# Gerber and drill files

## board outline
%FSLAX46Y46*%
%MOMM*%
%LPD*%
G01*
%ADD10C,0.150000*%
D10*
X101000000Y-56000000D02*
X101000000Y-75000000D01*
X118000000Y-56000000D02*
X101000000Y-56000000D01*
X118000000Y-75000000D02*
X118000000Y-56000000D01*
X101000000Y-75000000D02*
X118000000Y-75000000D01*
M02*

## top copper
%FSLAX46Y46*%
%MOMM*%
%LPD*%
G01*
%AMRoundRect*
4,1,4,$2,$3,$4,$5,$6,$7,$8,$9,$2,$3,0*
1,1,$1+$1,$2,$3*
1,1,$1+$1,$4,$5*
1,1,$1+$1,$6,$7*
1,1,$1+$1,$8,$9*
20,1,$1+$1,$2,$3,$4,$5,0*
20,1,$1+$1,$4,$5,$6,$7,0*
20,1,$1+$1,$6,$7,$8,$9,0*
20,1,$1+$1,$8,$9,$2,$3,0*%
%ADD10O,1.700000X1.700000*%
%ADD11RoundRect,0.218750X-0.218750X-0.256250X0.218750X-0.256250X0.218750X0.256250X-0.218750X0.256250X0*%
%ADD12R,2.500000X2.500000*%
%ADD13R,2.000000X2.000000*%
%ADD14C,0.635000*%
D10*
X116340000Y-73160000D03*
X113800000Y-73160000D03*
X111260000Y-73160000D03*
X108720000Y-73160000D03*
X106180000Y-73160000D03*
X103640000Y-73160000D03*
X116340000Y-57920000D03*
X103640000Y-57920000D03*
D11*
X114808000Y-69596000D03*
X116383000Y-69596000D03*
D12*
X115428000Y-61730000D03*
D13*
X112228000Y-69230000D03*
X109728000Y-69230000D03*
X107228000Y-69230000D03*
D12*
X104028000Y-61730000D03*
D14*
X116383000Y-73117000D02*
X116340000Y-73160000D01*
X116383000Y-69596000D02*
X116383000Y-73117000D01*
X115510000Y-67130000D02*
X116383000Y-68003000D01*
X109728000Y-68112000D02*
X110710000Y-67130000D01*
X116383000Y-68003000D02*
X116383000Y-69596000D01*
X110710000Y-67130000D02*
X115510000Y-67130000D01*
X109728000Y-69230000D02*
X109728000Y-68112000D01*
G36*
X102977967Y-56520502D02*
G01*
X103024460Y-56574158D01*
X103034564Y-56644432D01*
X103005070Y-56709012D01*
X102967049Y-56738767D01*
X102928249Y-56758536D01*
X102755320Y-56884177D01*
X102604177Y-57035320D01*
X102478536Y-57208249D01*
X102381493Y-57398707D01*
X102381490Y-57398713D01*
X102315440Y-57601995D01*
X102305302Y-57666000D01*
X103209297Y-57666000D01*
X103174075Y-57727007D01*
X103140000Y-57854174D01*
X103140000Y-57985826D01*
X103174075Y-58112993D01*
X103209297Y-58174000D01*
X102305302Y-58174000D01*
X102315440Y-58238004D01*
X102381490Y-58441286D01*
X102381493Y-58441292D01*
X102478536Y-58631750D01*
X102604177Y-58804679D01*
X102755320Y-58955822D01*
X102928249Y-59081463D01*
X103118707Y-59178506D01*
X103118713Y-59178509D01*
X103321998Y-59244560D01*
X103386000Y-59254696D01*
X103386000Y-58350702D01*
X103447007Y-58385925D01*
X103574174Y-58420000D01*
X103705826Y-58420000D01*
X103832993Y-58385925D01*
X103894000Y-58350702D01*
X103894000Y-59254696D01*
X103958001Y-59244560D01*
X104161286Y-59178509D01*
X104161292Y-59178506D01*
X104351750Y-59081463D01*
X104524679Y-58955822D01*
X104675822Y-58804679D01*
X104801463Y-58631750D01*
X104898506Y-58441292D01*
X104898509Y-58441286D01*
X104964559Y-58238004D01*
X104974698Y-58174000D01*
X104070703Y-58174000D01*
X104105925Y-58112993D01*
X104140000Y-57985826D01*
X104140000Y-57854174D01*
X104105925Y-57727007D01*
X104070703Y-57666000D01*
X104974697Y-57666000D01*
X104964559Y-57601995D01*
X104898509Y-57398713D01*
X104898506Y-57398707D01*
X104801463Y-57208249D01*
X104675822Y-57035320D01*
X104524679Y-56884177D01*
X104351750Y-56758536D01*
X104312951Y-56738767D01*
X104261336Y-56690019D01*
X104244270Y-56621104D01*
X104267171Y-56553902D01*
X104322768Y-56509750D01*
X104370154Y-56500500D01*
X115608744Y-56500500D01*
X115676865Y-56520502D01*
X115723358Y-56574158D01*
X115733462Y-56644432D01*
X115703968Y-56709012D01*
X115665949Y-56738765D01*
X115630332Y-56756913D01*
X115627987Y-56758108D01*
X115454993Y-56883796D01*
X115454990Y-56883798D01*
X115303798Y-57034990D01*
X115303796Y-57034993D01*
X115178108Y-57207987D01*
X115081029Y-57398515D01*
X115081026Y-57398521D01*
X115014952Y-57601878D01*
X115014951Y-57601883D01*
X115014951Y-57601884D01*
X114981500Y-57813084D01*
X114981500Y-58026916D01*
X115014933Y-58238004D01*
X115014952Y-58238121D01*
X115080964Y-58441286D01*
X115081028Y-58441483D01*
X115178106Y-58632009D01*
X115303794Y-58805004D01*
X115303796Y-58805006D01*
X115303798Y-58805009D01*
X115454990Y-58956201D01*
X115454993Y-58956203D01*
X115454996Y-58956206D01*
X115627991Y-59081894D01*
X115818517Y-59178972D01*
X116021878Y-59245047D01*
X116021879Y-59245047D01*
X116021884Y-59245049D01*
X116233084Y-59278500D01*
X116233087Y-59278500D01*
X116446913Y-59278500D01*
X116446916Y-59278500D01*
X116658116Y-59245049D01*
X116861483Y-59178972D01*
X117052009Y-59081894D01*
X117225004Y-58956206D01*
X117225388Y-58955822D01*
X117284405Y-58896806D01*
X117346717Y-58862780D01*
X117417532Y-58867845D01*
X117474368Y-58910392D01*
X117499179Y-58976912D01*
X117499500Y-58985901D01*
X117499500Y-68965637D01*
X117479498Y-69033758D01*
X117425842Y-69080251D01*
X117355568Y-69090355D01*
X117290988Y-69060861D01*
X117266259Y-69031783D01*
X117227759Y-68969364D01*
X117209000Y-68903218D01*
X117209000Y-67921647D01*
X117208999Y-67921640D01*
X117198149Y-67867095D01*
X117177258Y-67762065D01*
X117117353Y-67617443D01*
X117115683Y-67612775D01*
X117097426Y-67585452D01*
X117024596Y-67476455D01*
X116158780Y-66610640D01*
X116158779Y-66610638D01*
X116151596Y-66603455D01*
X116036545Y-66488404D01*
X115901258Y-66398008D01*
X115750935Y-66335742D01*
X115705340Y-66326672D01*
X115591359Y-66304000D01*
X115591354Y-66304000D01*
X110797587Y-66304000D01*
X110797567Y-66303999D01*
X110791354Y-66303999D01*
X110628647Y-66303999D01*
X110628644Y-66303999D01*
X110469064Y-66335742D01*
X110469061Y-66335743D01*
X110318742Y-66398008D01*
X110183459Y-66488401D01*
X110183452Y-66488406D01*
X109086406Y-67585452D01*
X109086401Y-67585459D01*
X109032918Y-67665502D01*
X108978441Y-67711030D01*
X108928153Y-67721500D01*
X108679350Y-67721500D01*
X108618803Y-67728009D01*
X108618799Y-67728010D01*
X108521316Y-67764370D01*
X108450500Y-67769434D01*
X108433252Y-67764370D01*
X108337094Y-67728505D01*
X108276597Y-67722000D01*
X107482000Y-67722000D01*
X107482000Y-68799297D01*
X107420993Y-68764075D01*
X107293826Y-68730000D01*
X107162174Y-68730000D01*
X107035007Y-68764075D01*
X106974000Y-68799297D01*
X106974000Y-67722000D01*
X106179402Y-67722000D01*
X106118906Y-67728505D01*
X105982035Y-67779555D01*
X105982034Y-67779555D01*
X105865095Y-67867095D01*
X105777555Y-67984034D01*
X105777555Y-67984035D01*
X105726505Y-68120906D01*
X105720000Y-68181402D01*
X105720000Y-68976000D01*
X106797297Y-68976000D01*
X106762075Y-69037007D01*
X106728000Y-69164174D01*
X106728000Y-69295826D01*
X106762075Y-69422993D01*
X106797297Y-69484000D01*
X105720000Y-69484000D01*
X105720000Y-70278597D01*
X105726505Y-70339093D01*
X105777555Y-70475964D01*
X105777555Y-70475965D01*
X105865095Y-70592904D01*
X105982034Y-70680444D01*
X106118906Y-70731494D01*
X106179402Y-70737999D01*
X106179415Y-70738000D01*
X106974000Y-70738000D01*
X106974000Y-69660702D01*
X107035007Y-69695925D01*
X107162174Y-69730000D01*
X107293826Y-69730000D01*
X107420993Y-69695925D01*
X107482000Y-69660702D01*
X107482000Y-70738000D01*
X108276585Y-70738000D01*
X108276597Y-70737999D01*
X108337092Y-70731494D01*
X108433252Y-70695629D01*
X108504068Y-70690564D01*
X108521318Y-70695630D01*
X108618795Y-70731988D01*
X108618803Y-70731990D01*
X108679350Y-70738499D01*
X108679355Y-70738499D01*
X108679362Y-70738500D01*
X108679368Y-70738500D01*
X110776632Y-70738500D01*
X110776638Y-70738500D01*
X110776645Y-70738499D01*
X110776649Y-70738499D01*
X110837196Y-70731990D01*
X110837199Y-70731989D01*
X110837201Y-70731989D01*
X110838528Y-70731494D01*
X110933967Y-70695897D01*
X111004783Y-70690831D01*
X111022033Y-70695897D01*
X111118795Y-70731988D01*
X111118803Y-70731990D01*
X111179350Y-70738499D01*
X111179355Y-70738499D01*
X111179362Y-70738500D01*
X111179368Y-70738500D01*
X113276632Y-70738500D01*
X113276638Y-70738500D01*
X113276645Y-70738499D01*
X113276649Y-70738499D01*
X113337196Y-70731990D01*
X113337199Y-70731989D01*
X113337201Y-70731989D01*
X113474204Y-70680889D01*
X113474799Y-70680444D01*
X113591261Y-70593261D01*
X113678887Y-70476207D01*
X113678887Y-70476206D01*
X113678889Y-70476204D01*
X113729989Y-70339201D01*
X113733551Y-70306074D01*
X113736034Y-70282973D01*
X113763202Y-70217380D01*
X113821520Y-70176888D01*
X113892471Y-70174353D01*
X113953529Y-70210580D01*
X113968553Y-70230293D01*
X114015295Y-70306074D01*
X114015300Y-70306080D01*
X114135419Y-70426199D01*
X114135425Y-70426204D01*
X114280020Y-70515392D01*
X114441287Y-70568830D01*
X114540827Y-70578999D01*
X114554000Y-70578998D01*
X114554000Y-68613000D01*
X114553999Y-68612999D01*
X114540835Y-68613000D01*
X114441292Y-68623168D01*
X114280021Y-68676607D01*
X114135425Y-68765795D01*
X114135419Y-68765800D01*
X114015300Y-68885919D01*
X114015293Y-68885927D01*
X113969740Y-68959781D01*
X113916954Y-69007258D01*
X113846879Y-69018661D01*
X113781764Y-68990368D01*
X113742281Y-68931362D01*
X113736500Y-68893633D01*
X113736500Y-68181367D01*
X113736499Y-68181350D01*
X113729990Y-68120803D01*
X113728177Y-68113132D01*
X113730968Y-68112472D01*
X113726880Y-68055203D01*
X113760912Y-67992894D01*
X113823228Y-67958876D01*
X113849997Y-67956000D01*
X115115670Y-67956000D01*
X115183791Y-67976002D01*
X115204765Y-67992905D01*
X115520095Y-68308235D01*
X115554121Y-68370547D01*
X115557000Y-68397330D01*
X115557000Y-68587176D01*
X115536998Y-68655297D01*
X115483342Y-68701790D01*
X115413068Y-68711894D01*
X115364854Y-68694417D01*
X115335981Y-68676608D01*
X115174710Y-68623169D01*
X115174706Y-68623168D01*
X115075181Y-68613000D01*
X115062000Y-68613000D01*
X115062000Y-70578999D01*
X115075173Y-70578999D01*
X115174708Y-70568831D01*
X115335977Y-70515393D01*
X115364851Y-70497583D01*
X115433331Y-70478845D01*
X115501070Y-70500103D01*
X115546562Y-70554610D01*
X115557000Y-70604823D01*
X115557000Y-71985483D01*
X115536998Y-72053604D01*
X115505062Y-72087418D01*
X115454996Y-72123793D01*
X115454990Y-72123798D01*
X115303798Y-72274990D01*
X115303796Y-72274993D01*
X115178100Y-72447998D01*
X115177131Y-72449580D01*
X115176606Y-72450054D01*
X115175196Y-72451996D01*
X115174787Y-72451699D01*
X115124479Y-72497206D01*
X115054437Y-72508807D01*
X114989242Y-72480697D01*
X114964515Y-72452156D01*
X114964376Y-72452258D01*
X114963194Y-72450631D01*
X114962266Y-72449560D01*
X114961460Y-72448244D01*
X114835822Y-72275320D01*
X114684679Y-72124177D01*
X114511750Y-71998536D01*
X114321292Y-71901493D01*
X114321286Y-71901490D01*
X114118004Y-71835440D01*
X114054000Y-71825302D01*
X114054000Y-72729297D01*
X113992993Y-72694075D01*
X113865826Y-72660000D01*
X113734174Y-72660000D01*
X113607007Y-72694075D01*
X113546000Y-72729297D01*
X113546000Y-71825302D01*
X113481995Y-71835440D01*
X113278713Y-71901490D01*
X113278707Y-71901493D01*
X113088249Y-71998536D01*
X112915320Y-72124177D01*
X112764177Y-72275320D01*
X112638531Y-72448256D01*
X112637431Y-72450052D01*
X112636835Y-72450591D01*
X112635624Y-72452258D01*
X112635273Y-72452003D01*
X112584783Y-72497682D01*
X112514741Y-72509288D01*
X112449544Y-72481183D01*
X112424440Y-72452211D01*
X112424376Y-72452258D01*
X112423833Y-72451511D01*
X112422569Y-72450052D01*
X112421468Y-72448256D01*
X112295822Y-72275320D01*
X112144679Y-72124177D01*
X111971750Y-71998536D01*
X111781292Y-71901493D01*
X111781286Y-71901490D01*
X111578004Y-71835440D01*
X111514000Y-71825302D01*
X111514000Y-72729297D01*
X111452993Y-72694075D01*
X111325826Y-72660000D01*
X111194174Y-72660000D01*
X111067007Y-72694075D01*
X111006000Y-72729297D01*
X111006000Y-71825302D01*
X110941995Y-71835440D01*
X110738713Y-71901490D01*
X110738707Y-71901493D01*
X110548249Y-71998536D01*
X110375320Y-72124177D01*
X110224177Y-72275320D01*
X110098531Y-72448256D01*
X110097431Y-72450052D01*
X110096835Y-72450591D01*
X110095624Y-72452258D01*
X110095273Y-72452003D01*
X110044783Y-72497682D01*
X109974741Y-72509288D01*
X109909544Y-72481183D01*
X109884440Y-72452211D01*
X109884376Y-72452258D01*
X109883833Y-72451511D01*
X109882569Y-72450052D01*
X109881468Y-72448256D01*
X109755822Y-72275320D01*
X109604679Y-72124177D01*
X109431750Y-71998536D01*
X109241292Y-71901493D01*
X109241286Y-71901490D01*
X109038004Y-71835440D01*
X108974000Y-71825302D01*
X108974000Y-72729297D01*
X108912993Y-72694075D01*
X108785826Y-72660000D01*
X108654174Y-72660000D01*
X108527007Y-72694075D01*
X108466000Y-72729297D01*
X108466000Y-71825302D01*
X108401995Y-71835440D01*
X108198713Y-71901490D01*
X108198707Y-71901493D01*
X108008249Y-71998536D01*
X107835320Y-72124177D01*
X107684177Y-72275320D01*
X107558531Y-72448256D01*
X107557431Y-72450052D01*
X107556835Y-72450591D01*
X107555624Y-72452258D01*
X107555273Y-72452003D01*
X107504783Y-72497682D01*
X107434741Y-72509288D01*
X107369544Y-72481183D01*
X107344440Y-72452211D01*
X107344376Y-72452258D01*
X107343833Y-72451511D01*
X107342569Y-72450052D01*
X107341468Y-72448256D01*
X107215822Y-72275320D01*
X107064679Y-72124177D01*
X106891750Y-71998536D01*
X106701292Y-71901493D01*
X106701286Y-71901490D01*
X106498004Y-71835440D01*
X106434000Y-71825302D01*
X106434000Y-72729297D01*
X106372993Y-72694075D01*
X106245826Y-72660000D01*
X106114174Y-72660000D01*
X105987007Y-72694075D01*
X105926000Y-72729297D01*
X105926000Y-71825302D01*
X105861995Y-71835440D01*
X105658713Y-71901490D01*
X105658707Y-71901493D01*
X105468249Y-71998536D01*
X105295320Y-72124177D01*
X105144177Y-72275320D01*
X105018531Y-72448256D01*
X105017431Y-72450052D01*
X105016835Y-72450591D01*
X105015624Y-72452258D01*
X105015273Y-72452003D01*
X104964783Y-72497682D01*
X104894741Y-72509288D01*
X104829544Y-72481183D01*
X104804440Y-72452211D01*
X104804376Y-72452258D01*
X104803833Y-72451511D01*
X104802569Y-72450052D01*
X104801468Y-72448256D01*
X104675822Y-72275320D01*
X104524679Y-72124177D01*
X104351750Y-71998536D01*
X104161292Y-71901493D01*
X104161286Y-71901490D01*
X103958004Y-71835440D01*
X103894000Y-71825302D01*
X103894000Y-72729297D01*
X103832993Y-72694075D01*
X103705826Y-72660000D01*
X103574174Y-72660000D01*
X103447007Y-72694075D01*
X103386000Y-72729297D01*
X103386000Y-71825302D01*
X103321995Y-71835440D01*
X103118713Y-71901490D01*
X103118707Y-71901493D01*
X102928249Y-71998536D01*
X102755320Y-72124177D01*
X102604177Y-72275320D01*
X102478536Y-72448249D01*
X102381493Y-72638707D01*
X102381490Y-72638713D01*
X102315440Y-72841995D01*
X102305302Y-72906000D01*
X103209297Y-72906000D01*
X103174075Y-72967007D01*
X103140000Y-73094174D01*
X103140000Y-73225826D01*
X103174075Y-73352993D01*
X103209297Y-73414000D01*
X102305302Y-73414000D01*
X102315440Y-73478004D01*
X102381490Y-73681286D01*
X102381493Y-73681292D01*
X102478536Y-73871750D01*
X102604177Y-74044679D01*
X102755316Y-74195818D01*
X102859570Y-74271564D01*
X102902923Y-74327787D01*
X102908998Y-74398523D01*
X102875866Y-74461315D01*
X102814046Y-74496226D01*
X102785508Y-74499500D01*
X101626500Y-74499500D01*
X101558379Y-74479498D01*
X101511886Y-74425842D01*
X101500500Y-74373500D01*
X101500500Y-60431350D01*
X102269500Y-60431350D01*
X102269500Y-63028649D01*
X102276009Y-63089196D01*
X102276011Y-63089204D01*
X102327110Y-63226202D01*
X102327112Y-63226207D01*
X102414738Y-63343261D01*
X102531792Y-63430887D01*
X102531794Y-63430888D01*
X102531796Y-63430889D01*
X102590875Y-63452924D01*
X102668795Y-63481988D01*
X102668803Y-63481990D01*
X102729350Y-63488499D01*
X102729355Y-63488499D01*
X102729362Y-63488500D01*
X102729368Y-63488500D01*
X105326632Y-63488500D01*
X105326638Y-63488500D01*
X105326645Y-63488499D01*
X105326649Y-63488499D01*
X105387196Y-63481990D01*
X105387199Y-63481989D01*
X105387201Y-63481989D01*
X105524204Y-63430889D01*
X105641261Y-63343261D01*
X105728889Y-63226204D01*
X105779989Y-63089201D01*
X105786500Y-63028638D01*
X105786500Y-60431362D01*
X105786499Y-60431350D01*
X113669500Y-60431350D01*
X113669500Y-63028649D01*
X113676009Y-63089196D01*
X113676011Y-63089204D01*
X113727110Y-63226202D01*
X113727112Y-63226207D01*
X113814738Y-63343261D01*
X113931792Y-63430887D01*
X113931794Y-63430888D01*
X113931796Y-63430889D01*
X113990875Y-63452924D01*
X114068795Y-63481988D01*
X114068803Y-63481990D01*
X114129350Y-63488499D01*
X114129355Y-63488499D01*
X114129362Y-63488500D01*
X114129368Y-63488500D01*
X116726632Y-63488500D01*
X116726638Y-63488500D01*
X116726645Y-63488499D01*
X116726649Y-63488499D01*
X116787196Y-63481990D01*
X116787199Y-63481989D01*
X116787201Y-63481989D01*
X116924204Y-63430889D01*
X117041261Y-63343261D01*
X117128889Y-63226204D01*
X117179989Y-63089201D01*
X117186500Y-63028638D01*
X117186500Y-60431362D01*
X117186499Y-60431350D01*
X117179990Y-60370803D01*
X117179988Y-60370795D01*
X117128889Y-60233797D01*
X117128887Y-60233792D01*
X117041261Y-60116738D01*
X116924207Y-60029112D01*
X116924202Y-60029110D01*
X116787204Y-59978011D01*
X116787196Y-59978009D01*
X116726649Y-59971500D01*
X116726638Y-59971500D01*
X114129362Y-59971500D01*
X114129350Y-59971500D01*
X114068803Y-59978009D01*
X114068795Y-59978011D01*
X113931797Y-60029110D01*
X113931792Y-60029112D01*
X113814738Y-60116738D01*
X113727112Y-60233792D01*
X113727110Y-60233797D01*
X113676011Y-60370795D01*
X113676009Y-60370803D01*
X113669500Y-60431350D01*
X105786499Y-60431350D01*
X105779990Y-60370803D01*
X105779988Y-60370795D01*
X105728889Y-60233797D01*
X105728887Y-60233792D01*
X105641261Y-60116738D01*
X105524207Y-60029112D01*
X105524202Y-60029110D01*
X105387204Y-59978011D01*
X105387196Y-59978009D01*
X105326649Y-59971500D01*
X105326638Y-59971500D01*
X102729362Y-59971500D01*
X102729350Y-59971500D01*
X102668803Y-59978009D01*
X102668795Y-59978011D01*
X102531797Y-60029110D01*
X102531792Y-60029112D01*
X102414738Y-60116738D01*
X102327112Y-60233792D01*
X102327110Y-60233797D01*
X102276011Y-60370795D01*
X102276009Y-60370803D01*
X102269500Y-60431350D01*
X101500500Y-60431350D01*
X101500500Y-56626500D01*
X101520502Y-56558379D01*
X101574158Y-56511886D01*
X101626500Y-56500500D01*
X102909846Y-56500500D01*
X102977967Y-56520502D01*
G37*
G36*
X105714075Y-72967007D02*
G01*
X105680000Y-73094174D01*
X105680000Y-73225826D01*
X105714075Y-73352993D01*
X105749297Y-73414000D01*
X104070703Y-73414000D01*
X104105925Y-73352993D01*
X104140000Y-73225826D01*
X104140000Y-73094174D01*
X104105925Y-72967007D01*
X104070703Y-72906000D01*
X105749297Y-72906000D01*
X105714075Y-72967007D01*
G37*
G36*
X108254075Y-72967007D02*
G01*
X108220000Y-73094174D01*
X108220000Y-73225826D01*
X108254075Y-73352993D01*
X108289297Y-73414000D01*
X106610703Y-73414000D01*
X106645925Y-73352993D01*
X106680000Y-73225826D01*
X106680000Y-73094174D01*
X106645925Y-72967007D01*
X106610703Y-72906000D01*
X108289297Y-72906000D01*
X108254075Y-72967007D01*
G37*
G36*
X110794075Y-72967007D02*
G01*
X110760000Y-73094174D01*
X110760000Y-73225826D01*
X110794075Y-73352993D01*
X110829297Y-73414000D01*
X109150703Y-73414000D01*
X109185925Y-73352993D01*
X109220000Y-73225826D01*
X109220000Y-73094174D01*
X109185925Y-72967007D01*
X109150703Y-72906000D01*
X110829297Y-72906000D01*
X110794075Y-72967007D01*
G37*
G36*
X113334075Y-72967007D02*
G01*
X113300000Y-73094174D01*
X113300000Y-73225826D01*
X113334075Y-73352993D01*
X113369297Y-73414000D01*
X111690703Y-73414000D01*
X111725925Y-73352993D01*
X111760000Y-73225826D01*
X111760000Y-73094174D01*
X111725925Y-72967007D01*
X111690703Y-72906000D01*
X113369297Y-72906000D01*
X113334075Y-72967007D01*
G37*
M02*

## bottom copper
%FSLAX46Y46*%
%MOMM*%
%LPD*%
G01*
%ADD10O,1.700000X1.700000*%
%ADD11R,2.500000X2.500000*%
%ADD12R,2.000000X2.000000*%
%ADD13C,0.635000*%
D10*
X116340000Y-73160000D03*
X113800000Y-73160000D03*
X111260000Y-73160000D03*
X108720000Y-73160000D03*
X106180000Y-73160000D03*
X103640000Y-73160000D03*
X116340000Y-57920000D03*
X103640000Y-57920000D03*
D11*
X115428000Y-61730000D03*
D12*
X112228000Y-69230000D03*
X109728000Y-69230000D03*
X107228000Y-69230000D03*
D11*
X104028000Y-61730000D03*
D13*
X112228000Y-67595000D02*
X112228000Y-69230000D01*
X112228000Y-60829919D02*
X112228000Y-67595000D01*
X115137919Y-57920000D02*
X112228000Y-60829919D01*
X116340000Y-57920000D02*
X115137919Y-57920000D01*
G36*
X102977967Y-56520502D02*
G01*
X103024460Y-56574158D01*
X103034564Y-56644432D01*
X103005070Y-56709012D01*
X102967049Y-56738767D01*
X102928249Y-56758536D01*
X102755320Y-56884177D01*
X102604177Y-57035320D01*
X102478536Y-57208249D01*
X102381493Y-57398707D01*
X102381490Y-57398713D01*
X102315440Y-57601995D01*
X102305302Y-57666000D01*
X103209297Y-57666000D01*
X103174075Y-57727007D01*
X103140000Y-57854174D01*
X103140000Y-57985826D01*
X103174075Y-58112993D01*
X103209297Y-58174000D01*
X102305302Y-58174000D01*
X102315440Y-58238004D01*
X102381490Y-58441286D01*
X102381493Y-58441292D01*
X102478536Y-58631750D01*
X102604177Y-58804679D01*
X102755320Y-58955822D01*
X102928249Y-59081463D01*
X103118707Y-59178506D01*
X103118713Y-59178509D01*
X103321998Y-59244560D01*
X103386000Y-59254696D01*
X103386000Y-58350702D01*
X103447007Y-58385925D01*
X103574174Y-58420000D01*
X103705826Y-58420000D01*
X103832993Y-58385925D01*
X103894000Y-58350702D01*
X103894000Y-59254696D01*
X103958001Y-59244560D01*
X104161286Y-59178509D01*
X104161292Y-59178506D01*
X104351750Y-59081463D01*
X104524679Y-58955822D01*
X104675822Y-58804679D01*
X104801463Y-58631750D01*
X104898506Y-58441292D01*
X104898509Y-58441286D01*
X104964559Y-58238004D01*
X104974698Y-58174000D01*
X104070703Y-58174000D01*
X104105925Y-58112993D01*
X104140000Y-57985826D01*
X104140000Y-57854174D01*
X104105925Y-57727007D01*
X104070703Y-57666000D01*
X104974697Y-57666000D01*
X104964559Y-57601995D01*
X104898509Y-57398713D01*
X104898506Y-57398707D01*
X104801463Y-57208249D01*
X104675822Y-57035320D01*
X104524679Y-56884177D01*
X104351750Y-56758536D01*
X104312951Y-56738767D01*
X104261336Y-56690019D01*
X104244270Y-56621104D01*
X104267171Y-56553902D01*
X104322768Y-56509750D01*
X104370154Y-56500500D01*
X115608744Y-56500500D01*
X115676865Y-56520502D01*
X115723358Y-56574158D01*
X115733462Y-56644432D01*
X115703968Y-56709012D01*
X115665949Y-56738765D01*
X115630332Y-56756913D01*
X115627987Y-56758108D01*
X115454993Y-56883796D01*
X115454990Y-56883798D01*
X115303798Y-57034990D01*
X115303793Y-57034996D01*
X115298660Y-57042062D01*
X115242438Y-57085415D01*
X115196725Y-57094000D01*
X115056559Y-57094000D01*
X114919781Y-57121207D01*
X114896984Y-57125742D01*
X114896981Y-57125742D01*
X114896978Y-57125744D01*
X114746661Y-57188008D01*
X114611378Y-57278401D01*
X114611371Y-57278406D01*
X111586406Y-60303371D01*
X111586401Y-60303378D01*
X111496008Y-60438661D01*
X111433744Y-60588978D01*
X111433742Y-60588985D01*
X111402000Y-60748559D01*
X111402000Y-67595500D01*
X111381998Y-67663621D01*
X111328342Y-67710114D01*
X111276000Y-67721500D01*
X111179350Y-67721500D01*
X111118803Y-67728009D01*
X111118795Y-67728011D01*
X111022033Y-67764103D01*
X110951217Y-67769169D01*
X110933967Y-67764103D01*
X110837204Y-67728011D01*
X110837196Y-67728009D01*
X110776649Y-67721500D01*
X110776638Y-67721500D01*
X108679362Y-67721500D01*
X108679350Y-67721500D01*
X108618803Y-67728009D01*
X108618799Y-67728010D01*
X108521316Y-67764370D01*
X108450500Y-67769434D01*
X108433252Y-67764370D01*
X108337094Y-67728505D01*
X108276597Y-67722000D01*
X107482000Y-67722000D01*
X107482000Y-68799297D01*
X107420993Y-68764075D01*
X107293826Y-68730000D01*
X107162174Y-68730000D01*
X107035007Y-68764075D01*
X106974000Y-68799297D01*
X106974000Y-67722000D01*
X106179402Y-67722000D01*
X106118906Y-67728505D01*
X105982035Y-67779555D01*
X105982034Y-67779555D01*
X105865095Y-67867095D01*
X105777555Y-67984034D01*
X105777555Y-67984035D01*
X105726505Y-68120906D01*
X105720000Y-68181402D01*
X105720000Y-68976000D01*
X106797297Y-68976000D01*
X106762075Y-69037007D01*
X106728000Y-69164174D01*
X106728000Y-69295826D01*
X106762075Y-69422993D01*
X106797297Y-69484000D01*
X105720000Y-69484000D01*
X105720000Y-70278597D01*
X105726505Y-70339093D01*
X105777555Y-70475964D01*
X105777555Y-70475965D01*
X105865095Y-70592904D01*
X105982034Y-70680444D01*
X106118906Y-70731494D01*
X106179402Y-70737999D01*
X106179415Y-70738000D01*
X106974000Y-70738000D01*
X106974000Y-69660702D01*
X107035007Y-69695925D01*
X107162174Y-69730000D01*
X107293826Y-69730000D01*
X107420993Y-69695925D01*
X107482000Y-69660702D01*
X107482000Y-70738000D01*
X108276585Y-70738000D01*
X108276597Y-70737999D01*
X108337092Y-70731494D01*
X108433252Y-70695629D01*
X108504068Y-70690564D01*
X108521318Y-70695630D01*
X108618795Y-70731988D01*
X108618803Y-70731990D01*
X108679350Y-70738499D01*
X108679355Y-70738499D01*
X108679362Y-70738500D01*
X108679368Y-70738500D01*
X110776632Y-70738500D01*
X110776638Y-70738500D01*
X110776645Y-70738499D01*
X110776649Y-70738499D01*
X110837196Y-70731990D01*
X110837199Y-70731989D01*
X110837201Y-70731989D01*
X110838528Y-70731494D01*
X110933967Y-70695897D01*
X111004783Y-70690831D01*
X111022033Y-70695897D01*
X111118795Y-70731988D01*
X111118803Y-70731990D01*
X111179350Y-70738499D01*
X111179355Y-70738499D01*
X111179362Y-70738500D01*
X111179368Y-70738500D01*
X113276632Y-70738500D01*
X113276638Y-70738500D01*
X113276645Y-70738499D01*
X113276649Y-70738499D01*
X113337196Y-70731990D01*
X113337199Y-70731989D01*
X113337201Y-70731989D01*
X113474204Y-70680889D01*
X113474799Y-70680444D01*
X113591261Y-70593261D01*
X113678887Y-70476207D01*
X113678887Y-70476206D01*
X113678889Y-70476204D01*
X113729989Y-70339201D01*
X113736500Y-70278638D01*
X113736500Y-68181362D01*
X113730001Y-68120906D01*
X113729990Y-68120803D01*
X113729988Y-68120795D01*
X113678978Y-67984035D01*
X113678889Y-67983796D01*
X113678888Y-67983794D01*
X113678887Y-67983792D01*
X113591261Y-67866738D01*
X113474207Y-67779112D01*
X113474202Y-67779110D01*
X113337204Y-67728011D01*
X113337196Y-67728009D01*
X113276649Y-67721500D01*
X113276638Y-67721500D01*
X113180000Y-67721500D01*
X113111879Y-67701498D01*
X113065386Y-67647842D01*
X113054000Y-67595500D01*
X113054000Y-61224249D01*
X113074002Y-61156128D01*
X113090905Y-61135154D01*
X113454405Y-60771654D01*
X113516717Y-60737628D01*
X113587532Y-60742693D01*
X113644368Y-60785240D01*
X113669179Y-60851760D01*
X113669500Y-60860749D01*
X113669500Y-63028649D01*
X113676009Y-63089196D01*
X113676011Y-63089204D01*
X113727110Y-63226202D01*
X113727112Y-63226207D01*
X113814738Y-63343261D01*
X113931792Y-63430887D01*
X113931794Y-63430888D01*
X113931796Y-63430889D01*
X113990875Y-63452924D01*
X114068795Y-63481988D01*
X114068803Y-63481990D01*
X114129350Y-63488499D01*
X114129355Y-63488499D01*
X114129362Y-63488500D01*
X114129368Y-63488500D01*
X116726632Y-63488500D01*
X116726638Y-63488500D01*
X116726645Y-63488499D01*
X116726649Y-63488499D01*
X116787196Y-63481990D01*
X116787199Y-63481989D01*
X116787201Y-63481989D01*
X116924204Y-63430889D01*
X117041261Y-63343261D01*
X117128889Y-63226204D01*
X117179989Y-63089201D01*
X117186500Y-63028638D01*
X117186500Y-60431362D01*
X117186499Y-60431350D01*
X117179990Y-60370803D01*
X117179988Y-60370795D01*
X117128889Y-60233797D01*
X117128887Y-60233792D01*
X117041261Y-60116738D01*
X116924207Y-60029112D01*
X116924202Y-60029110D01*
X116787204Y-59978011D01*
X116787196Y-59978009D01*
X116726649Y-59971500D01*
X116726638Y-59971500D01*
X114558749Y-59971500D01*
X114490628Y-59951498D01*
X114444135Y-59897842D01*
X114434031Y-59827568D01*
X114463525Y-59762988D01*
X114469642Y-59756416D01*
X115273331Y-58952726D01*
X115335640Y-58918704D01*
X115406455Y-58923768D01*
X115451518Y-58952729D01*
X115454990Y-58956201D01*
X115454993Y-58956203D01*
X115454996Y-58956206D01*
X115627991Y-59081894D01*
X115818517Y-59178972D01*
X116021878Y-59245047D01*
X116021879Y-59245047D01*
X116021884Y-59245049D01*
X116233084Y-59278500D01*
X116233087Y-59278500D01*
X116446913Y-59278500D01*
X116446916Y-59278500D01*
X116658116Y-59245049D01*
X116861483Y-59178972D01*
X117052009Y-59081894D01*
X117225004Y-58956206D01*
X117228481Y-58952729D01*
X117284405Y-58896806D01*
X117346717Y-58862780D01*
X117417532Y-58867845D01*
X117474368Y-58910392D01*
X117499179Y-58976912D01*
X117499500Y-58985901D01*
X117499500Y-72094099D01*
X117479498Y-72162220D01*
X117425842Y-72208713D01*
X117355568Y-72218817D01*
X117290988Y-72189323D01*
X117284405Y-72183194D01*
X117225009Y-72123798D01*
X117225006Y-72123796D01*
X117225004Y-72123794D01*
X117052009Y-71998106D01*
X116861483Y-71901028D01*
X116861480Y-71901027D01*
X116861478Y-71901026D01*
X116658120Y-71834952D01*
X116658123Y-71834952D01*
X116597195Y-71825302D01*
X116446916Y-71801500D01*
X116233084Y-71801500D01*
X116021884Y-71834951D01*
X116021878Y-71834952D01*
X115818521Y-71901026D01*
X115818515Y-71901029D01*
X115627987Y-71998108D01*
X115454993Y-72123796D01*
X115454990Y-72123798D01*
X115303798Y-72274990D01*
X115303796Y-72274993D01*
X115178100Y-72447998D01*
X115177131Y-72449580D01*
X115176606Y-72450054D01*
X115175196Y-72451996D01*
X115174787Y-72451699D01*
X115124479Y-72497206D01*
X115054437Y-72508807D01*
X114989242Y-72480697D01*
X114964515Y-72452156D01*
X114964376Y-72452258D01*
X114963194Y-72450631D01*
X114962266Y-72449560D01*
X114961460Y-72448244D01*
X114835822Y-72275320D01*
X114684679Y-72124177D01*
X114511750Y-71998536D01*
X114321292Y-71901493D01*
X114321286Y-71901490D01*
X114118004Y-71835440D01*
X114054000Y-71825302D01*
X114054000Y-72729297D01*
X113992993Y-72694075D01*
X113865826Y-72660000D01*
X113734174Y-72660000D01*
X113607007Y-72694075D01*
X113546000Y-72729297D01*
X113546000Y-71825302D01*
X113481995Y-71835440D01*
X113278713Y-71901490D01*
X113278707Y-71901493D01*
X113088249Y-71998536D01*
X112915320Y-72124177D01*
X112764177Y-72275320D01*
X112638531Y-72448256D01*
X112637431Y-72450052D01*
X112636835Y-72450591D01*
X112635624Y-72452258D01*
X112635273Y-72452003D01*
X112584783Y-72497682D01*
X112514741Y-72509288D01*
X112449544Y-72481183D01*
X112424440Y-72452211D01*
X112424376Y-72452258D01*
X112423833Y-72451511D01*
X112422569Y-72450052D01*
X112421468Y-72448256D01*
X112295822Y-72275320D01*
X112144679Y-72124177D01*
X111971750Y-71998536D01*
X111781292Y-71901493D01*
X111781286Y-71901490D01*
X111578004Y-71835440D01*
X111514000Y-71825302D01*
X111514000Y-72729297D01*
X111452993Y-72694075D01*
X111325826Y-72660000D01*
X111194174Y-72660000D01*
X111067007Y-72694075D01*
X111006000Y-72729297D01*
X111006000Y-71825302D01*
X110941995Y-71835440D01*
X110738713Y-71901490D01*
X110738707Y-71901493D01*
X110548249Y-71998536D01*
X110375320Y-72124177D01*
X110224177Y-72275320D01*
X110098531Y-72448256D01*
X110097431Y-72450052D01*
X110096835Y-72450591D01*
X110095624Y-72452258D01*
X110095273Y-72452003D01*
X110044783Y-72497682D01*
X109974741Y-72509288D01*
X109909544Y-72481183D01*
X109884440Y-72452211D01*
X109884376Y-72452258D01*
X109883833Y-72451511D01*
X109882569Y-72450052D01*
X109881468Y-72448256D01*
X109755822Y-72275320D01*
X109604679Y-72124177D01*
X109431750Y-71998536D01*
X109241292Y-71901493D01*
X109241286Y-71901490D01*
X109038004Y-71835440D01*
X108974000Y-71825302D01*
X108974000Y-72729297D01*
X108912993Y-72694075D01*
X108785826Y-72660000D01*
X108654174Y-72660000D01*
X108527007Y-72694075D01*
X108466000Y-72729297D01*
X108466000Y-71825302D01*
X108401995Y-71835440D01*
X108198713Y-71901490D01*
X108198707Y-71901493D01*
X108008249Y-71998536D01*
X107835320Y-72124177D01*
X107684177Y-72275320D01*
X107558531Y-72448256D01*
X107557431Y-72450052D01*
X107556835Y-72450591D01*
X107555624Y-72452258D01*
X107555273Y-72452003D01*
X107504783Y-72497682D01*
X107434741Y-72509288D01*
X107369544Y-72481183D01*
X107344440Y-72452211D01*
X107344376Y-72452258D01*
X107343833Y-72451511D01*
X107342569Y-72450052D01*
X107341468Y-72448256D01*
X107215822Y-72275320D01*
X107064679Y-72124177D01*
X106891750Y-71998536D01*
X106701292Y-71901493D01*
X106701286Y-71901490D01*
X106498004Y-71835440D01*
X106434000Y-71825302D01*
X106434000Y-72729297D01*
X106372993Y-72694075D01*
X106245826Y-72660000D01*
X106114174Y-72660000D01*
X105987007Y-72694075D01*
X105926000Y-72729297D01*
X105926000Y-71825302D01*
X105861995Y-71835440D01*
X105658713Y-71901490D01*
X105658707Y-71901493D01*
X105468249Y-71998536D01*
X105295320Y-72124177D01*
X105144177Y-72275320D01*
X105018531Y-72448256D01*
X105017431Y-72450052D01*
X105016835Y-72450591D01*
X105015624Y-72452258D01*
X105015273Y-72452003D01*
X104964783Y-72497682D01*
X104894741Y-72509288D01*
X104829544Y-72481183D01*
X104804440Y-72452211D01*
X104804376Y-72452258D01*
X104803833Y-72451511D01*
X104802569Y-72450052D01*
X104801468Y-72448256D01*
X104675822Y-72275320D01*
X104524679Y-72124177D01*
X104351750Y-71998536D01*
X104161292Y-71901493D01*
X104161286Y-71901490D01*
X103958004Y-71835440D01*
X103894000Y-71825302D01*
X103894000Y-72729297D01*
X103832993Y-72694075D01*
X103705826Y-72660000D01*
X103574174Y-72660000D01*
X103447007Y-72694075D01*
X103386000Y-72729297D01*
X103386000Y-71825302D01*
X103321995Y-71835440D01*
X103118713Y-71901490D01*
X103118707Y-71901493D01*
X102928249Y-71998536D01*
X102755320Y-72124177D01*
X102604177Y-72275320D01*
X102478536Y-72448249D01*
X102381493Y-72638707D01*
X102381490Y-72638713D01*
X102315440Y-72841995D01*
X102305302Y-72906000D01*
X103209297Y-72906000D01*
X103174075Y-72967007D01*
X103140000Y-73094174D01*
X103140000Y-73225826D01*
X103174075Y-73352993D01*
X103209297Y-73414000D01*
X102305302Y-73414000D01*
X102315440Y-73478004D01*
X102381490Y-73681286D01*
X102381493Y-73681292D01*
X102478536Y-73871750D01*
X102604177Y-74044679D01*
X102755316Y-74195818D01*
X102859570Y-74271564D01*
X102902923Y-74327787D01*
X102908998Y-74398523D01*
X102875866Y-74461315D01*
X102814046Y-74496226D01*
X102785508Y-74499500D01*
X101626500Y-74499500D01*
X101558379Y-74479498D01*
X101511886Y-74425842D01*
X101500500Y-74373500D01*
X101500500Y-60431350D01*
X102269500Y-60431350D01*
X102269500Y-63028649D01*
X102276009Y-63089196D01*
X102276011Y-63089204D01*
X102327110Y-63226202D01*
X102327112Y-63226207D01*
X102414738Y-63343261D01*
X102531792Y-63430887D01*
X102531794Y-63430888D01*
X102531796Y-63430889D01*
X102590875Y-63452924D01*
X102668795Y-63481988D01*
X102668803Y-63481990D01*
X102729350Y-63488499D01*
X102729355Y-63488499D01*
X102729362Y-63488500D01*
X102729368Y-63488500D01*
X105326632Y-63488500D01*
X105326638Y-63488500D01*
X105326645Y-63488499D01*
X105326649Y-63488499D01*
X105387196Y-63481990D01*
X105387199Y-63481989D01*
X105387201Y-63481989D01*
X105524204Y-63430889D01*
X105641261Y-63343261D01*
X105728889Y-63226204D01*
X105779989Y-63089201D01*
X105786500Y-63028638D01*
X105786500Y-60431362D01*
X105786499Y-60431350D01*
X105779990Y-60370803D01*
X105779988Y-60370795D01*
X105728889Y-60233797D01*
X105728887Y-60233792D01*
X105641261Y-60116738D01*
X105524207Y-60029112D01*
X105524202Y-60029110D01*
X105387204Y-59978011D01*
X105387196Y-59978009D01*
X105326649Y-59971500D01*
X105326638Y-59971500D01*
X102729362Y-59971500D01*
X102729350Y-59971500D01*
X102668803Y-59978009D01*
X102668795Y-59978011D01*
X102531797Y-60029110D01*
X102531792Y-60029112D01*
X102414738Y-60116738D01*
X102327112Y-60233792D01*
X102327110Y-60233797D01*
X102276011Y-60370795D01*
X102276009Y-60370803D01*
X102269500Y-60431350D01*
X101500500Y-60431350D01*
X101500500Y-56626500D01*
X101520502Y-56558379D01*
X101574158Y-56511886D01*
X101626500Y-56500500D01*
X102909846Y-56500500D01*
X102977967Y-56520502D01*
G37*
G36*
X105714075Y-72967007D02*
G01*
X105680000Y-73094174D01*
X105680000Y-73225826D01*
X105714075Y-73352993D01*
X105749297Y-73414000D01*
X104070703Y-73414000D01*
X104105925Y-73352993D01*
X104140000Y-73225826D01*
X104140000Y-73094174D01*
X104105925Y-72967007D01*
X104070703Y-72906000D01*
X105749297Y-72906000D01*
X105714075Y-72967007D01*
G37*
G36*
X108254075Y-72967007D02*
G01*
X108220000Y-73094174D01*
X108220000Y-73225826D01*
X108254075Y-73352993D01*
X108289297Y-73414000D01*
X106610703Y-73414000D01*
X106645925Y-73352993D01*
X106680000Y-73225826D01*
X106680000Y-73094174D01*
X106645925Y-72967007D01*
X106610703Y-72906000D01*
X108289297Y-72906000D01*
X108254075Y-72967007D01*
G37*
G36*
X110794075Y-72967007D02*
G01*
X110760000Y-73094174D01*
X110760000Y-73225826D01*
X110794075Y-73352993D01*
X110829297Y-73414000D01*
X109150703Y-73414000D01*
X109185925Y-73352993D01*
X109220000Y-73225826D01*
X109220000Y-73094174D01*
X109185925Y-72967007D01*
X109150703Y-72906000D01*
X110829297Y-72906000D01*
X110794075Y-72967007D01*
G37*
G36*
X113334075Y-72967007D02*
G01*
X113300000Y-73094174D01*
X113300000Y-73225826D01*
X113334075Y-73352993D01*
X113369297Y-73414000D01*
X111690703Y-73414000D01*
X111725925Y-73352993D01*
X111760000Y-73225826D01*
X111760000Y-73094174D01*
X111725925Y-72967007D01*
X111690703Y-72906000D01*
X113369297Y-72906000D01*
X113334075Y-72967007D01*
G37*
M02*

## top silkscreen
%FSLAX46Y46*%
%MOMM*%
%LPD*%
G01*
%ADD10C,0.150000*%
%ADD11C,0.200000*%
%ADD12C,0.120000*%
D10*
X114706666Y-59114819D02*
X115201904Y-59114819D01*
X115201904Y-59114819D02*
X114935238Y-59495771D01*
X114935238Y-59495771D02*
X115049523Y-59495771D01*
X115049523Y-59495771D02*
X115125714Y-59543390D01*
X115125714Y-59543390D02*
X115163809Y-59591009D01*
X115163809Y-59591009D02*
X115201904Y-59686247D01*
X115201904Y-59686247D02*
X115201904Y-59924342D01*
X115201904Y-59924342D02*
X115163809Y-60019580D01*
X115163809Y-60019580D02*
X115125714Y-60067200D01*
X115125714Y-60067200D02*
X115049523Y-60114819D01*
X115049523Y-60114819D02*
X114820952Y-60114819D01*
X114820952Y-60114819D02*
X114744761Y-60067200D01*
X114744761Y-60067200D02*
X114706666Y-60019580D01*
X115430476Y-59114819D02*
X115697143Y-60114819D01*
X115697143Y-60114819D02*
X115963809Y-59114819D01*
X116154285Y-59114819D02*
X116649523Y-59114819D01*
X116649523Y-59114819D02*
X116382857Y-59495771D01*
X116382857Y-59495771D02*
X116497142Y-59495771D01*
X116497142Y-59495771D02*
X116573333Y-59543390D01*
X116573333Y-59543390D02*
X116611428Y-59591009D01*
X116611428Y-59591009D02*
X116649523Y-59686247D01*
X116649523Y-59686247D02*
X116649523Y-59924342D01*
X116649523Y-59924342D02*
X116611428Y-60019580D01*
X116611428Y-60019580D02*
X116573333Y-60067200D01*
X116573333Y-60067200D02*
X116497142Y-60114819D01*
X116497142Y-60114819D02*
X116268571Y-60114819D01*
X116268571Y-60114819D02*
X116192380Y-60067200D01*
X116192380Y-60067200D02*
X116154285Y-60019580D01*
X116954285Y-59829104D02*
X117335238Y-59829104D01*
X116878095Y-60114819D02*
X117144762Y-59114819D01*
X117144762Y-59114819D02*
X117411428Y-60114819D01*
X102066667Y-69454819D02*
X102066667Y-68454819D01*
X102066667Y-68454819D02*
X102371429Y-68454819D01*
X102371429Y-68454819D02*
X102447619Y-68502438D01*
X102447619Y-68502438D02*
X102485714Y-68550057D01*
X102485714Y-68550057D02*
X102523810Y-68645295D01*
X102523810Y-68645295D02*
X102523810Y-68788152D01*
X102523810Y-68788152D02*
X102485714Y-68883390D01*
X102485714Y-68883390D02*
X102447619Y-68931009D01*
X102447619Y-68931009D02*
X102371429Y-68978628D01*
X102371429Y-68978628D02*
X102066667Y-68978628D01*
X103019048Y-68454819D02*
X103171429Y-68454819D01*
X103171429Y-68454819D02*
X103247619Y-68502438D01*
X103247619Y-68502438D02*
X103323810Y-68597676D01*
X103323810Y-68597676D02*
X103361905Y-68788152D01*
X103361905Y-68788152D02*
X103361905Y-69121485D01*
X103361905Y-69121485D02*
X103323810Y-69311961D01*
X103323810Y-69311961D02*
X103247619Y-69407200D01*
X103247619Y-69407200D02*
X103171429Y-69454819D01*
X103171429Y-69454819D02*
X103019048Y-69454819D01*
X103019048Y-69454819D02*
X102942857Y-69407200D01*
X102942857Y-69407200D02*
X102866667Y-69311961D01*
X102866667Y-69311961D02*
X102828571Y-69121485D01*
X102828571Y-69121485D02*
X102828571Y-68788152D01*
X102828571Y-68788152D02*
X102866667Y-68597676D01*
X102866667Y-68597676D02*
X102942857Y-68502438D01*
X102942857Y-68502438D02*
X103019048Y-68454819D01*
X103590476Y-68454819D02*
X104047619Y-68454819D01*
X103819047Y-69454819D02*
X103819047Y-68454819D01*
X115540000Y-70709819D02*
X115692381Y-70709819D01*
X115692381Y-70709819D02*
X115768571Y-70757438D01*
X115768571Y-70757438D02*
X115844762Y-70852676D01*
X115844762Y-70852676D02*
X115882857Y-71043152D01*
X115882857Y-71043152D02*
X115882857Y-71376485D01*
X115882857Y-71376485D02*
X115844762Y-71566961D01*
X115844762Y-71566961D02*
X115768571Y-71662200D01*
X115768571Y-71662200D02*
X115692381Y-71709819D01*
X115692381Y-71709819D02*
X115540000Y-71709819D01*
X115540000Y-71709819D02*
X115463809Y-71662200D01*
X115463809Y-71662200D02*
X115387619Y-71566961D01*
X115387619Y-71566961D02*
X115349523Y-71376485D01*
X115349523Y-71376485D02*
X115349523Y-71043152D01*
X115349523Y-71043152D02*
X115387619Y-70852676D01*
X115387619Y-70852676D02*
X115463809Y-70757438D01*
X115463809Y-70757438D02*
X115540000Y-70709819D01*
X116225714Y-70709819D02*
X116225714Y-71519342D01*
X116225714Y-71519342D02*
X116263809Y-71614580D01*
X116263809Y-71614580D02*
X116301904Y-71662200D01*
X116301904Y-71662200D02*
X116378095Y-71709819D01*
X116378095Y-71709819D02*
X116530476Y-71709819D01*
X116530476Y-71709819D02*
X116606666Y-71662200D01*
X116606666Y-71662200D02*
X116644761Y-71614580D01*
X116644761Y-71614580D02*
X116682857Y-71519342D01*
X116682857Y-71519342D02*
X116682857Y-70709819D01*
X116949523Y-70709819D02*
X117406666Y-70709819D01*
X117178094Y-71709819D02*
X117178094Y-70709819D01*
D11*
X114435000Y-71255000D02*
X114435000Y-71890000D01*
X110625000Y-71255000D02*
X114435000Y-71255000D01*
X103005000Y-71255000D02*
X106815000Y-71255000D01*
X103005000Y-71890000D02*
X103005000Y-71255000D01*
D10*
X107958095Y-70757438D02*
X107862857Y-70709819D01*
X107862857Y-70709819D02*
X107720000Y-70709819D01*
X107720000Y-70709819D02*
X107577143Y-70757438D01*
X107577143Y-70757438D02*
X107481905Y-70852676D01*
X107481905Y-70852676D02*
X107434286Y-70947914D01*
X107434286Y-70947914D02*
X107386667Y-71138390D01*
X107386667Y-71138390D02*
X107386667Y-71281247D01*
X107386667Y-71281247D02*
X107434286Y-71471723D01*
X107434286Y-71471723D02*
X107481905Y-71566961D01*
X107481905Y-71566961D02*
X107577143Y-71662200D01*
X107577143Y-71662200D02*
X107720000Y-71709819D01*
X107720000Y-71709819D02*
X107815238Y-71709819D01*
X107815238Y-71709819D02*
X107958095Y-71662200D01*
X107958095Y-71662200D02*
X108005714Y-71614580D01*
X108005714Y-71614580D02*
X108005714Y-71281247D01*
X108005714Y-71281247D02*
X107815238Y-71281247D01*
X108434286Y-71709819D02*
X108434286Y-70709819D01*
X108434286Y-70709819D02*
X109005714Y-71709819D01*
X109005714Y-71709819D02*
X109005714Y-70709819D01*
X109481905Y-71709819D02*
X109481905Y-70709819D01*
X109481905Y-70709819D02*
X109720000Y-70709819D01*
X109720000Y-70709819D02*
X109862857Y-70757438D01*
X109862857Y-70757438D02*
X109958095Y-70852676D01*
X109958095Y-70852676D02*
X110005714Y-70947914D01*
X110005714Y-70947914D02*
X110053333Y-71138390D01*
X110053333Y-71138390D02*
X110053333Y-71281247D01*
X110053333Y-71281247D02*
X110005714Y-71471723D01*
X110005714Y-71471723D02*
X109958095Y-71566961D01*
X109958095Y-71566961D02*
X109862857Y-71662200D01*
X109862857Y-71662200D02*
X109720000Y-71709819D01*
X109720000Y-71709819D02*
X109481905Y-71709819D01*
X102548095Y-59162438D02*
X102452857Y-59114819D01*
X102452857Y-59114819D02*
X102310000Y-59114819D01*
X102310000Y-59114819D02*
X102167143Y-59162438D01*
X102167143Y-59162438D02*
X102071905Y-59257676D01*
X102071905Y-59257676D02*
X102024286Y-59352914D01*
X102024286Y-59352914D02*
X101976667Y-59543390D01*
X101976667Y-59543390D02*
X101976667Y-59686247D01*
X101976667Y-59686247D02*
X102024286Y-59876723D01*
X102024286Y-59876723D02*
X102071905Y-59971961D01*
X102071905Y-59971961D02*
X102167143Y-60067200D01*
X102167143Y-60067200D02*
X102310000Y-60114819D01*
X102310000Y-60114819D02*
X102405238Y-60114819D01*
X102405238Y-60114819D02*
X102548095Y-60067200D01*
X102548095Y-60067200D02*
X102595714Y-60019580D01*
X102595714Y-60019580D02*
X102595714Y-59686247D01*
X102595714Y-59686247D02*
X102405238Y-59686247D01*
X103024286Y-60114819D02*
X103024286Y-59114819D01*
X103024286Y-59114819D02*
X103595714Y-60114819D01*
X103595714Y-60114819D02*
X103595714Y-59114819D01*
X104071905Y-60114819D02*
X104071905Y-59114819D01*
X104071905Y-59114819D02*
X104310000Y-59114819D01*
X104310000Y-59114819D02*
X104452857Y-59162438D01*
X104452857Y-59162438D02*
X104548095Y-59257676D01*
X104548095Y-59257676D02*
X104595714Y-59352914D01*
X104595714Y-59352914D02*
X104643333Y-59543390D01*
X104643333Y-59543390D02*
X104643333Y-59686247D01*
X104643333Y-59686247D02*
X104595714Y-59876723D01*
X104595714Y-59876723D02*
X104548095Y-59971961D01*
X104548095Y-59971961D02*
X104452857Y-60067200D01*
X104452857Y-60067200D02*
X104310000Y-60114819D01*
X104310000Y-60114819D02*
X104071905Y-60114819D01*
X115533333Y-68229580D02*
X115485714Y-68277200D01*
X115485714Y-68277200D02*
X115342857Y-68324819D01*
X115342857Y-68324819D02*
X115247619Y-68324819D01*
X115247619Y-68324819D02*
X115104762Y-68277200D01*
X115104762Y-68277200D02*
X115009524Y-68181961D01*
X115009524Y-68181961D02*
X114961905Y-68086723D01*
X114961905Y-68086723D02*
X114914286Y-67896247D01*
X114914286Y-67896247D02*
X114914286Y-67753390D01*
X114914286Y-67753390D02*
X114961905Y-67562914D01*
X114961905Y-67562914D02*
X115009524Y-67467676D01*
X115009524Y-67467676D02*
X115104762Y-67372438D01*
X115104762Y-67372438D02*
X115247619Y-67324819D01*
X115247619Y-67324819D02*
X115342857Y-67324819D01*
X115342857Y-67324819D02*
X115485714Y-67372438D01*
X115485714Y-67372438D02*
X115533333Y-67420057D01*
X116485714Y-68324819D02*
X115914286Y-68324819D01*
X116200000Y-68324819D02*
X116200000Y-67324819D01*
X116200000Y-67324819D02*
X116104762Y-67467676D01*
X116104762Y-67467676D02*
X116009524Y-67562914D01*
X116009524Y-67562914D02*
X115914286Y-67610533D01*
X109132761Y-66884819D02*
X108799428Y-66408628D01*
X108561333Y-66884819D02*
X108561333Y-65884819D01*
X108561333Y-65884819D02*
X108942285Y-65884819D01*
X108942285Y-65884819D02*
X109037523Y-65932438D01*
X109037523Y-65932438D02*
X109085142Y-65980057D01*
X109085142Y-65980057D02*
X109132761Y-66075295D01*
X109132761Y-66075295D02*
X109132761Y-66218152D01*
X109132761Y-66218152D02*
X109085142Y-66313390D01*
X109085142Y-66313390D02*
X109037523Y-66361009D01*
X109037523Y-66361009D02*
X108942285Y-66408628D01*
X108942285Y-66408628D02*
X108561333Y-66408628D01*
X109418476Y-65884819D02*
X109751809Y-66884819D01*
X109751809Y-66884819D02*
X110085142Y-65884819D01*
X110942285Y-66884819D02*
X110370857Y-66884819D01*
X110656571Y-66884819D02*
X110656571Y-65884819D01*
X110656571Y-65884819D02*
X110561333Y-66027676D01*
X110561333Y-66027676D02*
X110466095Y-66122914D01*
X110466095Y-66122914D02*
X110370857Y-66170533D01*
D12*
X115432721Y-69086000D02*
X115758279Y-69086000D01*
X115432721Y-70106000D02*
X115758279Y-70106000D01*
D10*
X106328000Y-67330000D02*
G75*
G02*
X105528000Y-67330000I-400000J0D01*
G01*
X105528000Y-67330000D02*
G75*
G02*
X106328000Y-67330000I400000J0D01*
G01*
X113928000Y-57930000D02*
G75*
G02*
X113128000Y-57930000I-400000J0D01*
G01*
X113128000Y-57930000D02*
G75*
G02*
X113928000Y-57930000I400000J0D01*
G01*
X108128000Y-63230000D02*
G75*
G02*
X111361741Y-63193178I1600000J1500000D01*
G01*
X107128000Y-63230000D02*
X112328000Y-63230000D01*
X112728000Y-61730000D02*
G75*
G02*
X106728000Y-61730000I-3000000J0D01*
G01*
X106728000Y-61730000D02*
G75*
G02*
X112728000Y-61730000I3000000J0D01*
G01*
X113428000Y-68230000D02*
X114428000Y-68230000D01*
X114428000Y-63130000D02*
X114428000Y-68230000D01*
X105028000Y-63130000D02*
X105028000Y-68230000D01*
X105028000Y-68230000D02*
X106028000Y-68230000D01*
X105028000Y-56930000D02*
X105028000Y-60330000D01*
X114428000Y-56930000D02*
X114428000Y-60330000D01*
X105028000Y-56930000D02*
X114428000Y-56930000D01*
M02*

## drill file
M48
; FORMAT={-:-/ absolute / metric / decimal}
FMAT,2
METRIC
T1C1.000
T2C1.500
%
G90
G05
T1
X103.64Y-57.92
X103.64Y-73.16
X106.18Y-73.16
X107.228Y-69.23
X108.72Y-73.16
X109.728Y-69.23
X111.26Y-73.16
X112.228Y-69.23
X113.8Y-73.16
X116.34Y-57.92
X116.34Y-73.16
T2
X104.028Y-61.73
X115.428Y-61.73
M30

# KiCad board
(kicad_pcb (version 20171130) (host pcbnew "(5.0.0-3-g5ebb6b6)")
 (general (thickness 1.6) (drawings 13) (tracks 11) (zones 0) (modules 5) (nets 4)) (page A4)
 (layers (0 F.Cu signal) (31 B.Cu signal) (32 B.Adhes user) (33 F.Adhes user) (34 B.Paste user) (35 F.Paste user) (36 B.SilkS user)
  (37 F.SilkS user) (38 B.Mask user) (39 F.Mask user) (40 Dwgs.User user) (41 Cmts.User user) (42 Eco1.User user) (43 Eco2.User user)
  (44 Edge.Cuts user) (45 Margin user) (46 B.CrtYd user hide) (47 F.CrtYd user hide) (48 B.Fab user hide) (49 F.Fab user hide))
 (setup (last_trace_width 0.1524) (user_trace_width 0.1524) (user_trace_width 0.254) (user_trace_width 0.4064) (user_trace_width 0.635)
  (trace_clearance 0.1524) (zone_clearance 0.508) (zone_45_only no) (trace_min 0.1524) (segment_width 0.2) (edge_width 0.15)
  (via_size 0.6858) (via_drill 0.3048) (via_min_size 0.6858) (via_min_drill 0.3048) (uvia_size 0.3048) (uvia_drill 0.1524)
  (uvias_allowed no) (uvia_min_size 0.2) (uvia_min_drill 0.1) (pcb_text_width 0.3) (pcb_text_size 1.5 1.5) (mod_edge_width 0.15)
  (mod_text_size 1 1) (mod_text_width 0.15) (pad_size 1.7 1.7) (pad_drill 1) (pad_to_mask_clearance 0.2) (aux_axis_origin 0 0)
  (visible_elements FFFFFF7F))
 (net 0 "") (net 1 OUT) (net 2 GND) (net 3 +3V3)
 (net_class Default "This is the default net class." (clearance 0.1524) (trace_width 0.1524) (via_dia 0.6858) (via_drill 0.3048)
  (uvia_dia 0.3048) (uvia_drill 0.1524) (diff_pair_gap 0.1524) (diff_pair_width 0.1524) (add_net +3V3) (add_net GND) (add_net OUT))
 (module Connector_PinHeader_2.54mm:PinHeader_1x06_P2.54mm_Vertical (layer B.Cu) (at 116.34 73.16 90)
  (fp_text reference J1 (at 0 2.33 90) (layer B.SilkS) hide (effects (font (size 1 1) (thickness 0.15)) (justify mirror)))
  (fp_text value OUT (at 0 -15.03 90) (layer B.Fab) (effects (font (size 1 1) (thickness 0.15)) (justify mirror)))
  (pad 1 thru_hole oval (at 0 0 90) (size 1.7 1.7) (drill 1) (layers *.Cu *.Mask) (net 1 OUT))
  (pad 2 thru_hole oval (at 0 -2.54 90) (size 1.7 1.7) (drill 1) (layers *.Cu *.Mask) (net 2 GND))
  (pad 3 thru_hole oval (at 0 -5.08 90) (size 1.7 1.7) (drill 1) (layers *.Cu *.Mask) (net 2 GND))
  (pad 4 thru_hole oval (at 0 -7.62 90) (size 1.7 1.7) (drill 1) (layers *.Cu *.Mask) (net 2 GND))
  (pad 5 thru_hole oval (at 0 -10.16 90) (size 1.7 1.7) (drill 1) (layers *.Cu *.Mask) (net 2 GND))
  (pad 6 thru_hole oval (at 0 -12.7 90) (size 1.7 1.7) (drill 1) (layers *.Cu *.Mask) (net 2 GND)))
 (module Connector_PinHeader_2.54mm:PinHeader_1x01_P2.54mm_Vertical (layer B.Cu) (at 116.34 57.92 90)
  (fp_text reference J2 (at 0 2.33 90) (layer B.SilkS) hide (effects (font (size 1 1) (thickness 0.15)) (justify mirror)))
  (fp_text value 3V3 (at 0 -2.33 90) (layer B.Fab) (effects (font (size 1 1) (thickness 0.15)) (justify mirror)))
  (pad 1 thru_hole oval (at 0 0 90) (size 1.7 1.7) (drill 1) (layers *.Cu *.Mask) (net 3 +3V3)))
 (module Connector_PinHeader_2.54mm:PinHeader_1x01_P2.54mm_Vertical (layer B.Cu) (at 103.64 57.92 270)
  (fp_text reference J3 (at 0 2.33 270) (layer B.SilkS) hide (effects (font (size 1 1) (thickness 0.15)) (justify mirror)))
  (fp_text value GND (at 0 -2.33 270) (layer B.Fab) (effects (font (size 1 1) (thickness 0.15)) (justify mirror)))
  (pad 1 thru_hole oval (at 0 0 270) (size 1.7 1.7) (drill 1) (layers *.Cu *.Mask) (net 2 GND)))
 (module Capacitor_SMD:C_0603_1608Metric (layer F.Cu) (at 115.5955 69.596)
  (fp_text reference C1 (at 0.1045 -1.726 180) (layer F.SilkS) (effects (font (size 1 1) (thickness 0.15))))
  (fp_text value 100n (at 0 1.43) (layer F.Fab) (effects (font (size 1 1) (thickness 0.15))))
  (fp_line (start -0.162779 -0.51) (end 0.162779 -0.51) (layer F.SilkS) (width 0.12))
  (fp_line (start -0.162779 0.51) (end 0.162779 0.51) (layer F.SilkS) (width 0.12))
  (pad 1 smd roundrect (at -0.7875 0) (size 0.875 0.95) (layers F.Cu F.Paste F.Mask) (roundrect_rratio 0.25) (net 2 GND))
  (pad 2 smd roundrect (at 0.7875 0) (size 0.875 0.95) (layers F.Cu F.Paste F.Mask) (roundrect_rratio 0.25) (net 1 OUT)))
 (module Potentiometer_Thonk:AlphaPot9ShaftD (layer F.Cu) (at 109.728 61.73)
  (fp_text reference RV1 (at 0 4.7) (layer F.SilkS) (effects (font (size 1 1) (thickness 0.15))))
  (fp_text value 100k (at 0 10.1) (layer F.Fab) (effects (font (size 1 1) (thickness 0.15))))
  (fp_circle (center -3.8 5.6) (end -4.2 5.6) (layer F.SilkS) (width 0.15))
  (fp_circle (center 3.8 -3.8) (end 4.2 -3.8) (layer F.SilkS) (width 0.15))
  (fp_arc (start 0 0) (end -1.6 1.5) (angle 265) (layer F.SilkS) (width 0.15))
  (fp_line (start -2.6 1.5) (end 2.6 1.5) (layer F.SilkS) (width 0.15))
  (fp_circle (center 0 0) (end 3 0) (layer F.SilkS) (width 0.15))
  (fp_line (start 3.7 6.5) (end 4.7 6.5) (layer F.SilkS) (width 0.15))
  (fp_line (start 4.7 1.4) (end 4.7 6.5) (layer F.SilkS) (width 0.15))
  (fp_line (start -4.7 1.4) (end -4.7 6.5) (layer F.SilkS) (width 0.15))
  (fp_line (start -4.7 6.5) (end -3.7 6.5) (layer F.SilkS) (width 0.15))
  (fp_line (start -4.7 -4.8) (end -4.7 -1.4) (layer F.SilkS) (width 0.15))
  (fp_line (start 4.7 -4.8) (end 4.7 -1.4) (layer F.SilkS) (width 0.15))
  (fp_line (start -4.7 -4.8) (end 4.7 -4.8) (layer F.SilkS) (width 0.15))
  (pad "" thru_hole rect (at 5.7 0) (size 2.5 2.5) (drill 1.5) (layers *.Cu *.Mask))
  (pad 3 thru_hole rect (at 2.5 7.5) (size 2 2) (drill 1) (layers *.Cu *.Mask) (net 3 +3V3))
  (pad 2 thru_hole rect (at 0 7.5) (size 2 2) (drill 1) (layers *.Cu *.Mask) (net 1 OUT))
  (pad 1 thru_hole rect (at -2.5 7.5) (size 2 2) (drill 1) (layers *.Cu *.Mask) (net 2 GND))
  (pad "" thru_hole rect (at -5.7 0) (size 2.5 2.5) (drill 1.5) (layers *.Cu *.Mask)))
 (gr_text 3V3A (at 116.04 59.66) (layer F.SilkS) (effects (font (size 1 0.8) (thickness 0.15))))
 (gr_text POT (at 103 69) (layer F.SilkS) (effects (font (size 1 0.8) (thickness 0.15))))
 (gr_line (start 101 56) (end 101 75) (layer Edge.Cuts) (width 0.15))
 (gr_line (start 118 56) (end 101 56) (layer Edge.Cuts) (width 0.15))
 (gr_line (start 118 75) (end 118 56) (layer Edge.Cuts) (width 0.15))
 (gr_line (start 101 75) (end 118 75) (layer Edge.Cuts) (width 0.15))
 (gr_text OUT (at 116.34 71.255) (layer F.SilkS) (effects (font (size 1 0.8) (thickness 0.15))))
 (gr_line (start 114.435 71.255) (end 114.435 71.89) (layer F.SilkS) (width 0.2))
 (gr_line (start 110.625 71.255) (end 114.435 71.255) (layer F.SilkS) (width 0.2))
 (gr_line (start 103.005 71.255) (end 106.815 71.255) (layer F.SilkS) (width 0.2))
 (gr_line (start 103.005 71.89) (end 103.005 71.255) (layer F.SilkS) (width 0.2))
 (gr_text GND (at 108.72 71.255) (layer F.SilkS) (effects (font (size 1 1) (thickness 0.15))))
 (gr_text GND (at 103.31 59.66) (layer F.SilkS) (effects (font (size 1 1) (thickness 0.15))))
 (segment (start 116.383 73.117) (end 116.34 73.16) (width 0.635) (layer F.Cu) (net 1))
 (segment (start 116.383 69.596) (end 116.383 73.117) (width 0.635) (layer F.Cu) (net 1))
 (segment (start 115.51 67.13) (end 116.383 68.003) (width 0.635) (layer F.Cu) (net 1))
 (segment (start 109.728 68.112) (end 110.71 67.13) (width 0.635) (layer F.Cu) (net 1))
 (segment (start 116.383 68.003) (end 116.383 69.596) (width 0.635) (layer F.Cu) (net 1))
 (segment (start 110.71 67.13) (end 115.51 67.13) (width 0.635) (layer F.Cu) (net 1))
 (segment (start 109.728 69.23) (end 109.728 68.112) (width 0.635) (layer F.Cu) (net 1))
 (segment (start 112.228 67.595) (end 112.228 69.23) (width 0.635) (layer B.Cu) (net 3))
 (segment (start 112.228 60.829919) (end 112.228 67.595) (width 0.635) (layer B.Cu) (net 3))
 (segment (start 115.137919 57.92) (end 112.228 60.829919) (width 0.635) (layer B.Cu) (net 3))
 (segment (start 116.34 57.92) (end 115.137919 57.92) (width 0.635) (layer B.Cu) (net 3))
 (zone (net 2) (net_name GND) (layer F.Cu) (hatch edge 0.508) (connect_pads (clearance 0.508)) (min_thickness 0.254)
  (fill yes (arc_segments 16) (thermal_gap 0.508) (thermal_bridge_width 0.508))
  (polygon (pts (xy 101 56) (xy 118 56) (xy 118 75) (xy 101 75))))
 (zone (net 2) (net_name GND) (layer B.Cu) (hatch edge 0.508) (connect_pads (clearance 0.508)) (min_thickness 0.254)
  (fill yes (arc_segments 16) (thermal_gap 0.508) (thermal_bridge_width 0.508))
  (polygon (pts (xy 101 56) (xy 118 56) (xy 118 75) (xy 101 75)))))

